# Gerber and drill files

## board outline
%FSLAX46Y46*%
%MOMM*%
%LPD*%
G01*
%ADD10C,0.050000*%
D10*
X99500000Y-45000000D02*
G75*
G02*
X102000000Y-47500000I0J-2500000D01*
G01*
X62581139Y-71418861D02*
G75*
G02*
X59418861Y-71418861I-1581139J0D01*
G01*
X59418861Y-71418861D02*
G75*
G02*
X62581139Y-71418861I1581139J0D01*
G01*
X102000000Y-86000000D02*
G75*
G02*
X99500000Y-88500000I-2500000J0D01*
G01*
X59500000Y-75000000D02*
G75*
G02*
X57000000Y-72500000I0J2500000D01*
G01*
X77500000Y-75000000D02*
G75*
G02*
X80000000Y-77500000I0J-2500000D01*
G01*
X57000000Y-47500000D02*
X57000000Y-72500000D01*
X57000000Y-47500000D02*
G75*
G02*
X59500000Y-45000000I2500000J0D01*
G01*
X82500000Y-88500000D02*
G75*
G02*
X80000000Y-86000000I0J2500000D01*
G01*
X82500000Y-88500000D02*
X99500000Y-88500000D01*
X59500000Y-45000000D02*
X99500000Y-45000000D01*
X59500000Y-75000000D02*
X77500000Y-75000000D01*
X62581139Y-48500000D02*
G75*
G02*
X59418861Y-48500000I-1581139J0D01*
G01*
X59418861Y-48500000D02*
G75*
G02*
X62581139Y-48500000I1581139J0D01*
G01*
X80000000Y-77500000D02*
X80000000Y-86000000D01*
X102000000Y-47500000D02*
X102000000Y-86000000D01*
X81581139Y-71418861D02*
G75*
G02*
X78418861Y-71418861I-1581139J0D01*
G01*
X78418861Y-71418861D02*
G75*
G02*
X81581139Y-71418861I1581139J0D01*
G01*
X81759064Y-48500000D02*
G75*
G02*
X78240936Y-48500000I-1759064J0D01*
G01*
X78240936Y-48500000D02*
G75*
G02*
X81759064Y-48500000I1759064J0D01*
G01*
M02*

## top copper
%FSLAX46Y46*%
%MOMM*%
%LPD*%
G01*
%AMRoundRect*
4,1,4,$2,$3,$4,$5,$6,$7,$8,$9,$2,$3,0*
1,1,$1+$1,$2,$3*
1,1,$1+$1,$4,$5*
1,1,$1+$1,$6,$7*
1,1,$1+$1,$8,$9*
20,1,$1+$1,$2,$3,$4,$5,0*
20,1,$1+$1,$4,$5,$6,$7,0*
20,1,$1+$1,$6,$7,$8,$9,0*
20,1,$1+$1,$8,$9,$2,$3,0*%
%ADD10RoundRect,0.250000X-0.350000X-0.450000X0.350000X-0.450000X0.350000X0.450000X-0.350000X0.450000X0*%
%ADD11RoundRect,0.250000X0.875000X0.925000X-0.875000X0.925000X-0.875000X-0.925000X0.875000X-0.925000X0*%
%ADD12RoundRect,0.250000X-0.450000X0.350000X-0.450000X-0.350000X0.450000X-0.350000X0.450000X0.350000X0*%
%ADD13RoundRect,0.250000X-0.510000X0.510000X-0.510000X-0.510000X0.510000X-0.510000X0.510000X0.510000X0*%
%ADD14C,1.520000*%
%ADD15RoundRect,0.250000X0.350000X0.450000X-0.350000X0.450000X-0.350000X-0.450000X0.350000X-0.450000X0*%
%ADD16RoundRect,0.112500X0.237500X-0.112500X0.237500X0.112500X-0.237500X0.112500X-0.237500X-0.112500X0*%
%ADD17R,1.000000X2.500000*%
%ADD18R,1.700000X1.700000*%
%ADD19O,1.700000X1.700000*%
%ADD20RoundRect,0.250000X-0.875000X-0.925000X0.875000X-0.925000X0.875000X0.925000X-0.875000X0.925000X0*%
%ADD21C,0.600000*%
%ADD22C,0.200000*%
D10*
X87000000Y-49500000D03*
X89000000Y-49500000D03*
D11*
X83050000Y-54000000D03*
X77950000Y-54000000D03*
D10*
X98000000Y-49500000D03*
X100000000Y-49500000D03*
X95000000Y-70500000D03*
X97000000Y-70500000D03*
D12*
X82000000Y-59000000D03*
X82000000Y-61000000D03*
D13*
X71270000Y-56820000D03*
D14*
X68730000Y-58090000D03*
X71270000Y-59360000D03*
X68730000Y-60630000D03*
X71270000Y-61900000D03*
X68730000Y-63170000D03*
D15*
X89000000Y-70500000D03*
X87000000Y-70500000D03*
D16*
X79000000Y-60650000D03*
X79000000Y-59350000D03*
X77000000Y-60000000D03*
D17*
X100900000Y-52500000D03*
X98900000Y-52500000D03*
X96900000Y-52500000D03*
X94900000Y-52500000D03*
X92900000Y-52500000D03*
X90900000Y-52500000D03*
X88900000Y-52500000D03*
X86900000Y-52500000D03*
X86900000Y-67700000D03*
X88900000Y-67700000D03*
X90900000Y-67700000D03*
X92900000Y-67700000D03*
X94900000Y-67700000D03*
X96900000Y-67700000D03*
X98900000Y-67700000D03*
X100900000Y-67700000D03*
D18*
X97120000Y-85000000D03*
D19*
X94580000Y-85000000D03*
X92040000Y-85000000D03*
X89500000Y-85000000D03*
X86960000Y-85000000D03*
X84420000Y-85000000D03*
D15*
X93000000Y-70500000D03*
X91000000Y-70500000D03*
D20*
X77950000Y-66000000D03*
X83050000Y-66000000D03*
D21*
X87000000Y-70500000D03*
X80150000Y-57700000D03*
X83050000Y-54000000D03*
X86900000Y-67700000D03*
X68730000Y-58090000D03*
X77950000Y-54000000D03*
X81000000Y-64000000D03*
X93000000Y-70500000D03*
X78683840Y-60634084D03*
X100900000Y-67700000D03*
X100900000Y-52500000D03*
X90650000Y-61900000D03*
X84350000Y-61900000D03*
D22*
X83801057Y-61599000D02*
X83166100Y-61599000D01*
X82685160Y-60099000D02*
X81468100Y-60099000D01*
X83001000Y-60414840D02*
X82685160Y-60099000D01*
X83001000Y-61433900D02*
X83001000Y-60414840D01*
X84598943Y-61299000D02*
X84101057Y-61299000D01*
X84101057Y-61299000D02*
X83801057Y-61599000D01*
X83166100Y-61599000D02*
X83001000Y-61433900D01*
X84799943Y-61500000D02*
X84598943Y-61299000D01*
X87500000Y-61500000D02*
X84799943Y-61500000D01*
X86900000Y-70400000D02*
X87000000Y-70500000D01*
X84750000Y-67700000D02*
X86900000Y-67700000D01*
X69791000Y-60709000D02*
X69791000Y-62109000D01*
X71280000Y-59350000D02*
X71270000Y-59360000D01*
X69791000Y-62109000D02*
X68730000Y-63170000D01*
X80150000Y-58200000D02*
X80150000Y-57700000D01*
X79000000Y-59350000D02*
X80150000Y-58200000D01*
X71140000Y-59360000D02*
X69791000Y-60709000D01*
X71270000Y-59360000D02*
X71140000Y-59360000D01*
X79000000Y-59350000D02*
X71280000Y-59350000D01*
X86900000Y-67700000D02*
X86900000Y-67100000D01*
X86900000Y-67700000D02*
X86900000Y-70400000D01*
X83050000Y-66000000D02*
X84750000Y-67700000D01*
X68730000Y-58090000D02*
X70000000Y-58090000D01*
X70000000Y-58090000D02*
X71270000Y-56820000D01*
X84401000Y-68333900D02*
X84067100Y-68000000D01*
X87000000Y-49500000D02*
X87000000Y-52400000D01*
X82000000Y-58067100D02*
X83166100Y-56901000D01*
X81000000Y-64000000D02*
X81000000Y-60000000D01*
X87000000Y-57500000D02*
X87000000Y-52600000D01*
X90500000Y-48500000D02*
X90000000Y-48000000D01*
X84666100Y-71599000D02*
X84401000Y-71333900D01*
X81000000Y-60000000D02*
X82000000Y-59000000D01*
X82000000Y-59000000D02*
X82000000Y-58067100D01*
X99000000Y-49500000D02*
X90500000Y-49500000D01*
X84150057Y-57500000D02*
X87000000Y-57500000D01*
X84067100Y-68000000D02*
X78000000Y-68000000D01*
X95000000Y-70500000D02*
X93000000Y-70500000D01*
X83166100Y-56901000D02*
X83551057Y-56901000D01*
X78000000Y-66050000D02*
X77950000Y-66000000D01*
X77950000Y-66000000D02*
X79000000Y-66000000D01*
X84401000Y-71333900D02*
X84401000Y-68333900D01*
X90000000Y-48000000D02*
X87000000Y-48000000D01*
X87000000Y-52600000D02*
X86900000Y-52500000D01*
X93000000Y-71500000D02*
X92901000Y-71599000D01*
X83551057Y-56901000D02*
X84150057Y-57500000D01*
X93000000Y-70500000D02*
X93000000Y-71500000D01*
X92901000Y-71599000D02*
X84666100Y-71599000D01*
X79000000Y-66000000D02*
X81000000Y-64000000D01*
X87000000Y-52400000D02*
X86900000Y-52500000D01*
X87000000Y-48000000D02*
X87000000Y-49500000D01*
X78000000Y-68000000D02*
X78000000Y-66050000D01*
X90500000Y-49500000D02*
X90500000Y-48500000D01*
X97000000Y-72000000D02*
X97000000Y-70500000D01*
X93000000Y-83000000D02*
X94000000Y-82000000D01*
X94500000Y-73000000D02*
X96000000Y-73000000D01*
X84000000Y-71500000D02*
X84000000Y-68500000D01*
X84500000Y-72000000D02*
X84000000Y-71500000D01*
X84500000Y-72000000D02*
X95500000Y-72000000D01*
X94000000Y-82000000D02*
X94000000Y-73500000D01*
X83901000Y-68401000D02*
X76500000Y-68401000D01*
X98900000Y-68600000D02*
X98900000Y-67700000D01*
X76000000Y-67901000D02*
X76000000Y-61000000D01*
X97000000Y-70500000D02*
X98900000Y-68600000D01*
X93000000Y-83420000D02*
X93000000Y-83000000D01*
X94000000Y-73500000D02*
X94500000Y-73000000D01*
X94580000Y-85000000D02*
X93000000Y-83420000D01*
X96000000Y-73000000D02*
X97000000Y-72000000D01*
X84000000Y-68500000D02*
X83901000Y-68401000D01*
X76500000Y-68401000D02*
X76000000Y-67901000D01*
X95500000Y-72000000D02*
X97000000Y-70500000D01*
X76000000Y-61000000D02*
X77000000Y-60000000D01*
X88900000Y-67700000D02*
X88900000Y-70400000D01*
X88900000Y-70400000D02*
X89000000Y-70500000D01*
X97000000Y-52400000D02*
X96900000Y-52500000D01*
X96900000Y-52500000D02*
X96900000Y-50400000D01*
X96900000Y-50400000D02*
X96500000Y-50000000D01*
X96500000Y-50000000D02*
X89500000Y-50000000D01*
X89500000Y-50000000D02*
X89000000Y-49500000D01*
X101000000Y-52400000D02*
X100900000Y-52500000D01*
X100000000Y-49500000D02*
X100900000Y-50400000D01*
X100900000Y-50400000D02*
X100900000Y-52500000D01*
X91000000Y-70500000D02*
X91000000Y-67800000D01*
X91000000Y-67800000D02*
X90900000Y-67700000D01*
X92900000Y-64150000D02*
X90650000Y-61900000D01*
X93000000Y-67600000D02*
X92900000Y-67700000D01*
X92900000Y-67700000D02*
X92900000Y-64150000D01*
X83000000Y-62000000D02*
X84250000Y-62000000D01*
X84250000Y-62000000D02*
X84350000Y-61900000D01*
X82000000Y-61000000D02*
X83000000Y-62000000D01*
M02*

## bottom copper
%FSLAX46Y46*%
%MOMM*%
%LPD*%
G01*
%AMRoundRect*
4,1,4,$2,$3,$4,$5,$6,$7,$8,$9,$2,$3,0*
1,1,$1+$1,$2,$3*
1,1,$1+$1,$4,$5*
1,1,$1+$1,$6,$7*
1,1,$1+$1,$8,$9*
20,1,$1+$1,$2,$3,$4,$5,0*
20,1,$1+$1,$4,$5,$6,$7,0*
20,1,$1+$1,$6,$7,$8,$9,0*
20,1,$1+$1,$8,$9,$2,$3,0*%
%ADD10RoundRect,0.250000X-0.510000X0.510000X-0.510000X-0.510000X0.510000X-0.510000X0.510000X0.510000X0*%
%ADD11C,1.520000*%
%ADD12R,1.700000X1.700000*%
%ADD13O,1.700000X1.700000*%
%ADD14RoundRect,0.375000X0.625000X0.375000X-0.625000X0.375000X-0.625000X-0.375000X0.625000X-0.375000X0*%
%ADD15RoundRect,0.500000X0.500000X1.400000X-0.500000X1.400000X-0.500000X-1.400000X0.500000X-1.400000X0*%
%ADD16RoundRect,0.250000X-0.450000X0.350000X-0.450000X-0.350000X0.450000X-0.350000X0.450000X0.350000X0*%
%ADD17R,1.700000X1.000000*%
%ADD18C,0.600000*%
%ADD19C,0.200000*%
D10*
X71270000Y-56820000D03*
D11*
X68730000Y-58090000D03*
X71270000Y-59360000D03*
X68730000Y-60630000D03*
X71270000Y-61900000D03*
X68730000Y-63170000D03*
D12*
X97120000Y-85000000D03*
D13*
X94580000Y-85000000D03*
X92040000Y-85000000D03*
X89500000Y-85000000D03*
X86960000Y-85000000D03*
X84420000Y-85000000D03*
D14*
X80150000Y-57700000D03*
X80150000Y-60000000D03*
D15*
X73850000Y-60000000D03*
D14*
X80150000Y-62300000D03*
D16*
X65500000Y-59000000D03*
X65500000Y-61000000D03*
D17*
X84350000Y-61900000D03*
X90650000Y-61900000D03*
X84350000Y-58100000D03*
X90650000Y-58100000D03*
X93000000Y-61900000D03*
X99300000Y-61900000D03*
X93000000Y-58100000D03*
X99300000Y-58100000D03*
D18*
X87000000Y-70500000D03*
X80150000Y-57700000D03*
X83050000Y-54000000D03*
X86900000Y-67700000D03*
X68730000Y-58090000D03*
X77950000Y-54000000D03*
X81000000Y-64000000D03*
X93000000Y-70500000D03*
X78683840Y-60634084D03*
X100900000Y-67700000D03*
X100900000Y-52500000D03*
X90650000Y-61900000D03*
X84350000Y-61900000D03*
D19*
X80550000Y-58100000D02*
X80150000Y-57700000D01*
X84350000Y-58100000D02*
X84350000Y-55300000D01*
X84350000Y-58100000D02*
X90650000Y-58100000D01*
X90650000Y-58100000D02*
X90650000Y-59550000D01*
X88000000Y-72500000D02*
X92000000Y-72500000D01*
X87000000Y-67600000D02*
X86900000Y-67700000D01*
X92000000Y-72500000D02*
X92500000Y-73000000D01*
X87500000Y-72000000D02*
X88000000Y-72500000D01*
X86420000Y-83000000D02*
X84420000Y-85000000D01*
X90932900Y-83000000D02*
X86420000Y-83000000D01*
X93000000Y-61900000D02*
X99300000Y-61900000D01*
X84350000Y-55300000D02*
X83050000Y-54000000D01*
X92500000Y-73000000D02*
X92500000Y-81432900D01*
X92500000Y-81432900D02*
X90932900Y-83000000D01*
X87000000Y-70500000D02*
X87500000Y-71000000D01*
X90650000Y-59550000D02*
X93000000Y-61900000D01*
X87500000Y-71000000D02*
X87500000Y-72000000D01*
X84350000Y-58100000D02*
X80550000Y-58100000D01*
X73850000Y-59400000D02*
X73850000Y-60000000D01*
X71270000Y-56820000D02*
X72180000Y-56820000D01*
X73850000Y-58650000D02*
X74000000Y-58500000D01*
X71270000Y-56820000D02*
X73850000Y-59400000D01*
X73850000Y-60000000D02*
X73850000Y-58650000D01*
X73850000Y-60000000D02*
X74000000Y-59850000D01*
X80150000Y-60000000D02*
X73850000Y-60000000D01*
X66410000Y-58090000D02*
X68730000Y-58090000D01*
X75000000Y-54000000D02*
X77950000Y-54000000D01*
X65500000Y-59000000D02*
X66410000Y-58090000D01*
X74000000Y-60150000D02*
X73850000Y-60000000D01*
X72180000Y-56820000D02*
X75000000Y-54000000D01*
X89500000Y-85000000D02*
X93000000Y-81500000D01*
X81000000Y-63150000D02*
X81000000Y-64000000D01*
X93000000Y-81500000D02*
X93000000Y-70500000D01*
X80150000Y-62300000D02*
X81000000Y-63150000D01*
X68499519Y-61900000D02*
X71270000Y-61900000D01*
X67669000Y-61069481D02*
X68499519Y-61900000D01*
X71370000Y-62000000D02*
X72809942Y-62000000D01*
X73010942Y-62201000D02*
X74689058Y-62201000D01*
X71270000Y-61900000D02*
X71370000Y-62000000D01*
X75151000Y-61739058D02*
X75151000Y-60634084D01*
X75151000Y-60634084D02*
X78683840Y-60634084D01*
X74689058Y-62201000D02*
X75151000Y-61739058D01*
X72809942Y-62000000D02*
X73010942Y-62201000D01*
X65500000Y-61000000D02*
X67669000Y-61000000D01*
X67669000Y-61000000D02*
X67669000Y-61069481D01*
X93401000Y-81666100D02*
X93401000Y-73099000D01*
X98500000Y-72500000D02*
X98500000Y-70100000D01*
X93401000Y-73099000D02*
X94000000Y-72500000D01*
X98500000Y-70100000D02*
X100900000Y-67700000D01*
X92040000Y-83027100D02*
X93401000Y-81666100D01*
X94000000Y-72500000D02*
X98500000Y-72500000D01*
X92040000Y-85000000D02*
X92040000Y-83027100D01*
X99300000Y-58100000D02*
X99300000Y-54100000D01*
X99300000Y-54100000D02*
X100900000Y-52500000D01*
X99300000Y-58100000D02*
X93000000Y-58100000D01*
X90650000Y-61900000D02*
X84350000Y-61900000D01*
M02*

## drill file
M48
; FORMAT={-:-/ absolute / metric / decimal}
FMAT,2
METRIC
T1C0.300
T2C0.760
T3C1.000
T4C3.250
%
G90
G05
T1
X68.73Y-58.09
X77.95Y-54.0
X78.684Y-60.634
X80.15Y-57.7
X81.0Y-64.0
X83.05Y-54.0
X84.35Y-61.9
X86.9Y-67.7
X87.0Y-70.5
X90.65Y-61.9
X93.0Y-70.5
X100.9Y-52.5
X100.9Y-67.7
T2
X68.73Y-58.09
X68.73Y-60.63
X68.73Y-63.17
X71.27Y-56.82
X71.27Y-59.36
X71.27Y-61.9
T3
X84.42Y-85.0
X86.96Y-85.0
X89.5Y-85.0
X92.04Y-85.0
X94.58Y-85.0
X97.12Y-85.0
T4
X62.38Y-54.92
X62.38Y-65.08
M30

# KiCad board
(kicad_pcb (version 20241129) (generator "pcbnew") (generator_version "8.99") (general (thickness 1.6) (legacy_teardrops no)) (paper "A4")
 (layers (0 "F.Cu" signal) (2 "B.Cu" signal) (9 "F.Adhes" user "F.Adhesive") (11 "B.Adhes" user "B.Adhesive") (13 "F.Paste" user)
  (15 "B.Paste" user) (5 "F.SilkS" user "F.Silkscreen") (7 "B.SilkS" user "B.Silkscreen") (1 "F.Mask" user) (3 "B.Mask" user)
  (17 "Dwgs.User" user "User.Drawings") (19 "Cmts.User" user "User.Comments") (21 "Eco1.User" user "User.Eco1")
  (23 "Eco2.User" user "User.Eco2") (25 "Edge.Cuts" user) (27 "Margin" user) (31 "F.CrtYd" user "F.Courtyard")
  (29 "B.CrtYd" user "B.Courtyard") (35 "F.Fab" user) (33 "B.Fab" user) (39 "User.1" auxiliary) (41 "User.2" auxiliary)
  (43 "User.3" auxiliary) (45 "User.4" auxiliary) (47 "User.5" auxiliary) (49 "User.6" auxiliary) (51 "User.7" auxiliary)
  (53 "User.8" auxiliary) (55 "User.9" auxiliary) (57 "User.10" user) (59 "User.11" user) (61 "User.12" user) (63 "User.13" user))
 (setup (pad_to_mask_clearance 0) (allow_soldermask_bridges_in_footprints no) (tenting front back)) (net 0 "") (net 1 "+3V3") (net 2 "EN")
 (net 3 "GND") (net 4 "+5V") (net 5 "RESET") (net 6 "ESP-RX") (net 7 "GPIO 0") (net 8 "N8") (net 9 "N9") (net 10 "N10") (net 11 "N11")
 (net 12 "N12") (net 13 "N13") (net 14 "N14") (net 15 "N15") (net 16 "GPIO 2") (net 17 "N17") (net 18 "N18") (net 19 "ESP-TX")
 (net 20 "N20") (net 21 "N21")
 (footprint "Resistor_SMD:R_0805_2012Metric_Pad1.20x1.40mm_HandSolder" (layer "F.Cu") (at 88 49.5)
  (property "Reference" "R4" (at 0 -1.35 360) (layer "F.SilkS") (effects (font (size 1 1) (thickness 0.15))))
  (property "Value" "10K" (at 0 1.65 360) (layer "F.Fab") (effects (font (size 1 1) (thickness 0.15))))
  (pad "1" smd roundrect (at -1 0) (size 1.2 1.4) (layers "F.Cu" "F.Mask" "F.Paste") (roundrect_rratio 0.208333) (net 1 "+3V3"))
  (pad "2" smd roundrect (at 1 0) (size 1.2 1.4) (layers "F.Cu" "F.Mask" "F.Paste") (roundrect_rratio 0.208333) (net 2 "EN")))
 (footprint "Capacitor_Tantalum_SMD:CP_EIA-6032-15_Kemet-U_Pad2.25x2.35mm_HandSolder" (layer "F.Cu") (at 80.5 54 180)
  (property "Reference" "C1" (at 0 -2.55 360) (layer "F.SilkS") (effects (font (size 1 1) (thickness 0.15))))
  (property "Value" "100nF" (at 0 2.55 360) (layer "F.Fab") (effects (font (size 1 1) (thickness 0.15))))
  (pad "1" smd roundrect (at -2.55 0 180) (size 2.25 2.35) (layers "F.Cu" "F.Mask" "F.Paste") (roundrect_rratio 0.111111) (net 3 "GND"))
  (pad "2" smd roundrect (at 2.55 0 180) (size 2.25 2.35) (layers "F.Cu" "F.Mask" "F.Paste") (roundrect_rratio 0.111111) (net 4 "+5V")))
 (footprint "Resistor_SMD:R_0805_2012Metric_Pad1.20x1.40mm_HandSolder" (layer "F.Cu") (at 99 49.5)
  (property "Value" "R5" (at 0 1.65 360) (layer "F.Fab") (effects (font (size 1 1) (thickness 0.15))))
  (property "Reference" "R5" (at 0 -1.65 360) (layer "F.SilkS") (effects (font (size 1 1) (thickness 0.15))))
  (pad "1" smd roundrect (at -1 0) (size 1.2 1.4) (layers "F.Cu" "F.Mask" "F.Paste") (roundrect_rratio 0.208333) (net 1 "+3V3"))
  (pad "2" smd roundrect (at 1 0) (size 1.2 1.4) (layers "F.Cu" "F.Mask" "F.Paste") (roundrect_rratio 0.208333) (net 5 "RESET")))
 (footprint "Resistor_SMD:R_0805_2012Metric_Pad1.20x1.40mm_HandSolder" (layer "F.Cu") (at 96 70.5)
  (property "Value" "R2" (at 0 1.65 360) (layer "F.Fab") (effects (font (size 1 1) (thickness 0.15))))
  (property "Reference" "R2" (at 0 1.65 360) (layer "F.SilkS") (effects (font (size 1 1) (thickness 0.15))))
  (pad "1" smd roundrect (at -1 0) (size 1.2 1.4) (layers "F.Cu" "F.Mask" "F.Paste") (roundrect_rratio 0.208333) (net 1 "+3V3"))
  (pad "2" smd roundrect (at 1 0) (size 1.2 1.4) (layers "F.Cu" "F.Mask" "F.Paste") (roundrect_rratio 0.208333) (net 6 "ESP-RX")))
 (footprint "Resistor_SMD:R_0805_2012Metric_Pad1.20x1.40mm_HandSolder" (layer "F.Cu") (at 82 60 -90)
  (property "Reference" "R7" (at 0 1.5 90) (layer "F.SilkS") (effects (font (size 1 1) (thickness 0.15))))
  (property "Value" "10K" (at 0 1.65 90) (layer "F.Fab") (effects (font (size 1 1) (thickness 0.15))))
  (pad "1" smd roundrect (at -1 0 270) (size 1.2 1.4) (layers "F.Cu" "F.Mask" "F.Paste") (roundrect_rratio 0.208333) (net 1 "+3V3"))
  (pad "2" smd roundrect (at 1 0 270) (size 1.2 1.4) (layers "F.Cu" "F.Mask" "F.Paste") (roundrect_rratio 0.208333) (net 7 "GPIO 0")))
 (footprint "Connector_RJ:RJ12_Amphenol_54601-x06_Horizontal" (layer "F.Cu") (at 71.27 56.82 -90)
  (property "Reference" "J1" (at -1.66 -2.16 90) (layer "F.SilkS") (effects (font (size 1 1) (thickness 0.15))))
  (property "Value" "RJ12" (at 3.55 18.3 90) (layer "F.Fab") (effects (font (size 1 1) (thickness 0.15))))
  (pad "" np_thru_hole circle (at -1.9 8.89 270) (size 3.25 3.25) (drill 3.25) (layers "*.Cu" "*.Mask"))
  (pad "" np_thru_hole circle (at 8.26 8.89 270) (size 3.25 3.25) (drill 3.25) (layers "*.Cu" "*.Mask"))
  (pad "1" thru_hole roundrect (at 0 0 270) (size 1.52 1.52) (drill 0.76) (layers "*.Cu" "*.Mask") (remove_unused_layers no)
   (roundrect_rratio 0.1644736842) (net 4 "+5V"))
  (pad "2" thru_hole circle (at 1.27 2.54 270) (size 1.52 1.52) (drill 0.76) (layers "*.Cu" "*.Mask") (remove_unused_layers no)
   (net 4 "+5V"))
  (pad "3" thru_hole circle (at 2.54 0 270) (size 1.52 1.52) (drill 0.76) (layers "*.Cu" "*.Mask") (remove_unused_layers no) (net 3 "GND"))
  (pad "4" thru_hole circle (at 3.81 2.54 270) (size 1.52 1.52) (drill 0.76) (layers "*.Cu" "*.Mask") (remove_unused_layers no) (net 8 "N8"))
  (pad "5" thru_hole circle (at 5.08 0 270) (size 1.52 1.52) (drill 0.76) (layers "*.Cu" "*.Mask") (remove_unused_layers no) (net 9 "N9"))
  (pad "6" thru_hole circle (at 6.35 2.54 270) (size 1.52 1.52) (drill 0.76) (layers "*.Cu" "*.Mask") (remove_unused_layers no)
   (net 3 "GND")))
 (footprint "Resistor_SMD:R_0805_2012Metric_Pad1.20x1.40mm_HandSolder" (layer "F.Cu") (at 88 70.5 180)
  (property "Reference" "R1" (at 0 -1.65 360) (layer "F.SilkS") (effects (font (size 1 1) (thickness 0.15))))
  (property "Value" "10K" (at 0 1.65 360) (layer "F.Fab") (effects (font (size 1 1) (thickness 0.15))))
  (pad "1" smd roundrect (at -1 0 180) (size 1.2 1.4) (layers "F.Cu" "F.Mask" "F.Paste") (roundrect_rratio 0.208333) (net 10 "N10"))
  (pad "2" smd roundrect (at 1 0 180) (size 1.2 1.4) (layers "F.Cu" "F.Mask" "F.Paste") (roundrect_rratio 0.208333) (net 3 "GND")))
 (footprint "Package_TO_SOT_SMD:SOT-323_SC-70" (layer "F.Cu") (at 78 60 180)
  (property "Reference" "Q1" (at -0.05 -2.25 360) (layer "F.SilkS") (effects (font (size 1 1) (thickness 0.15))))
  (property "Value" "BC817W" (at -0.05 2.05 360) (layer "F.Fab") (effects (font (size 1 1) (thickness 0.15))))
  (pad "1" smd roundrect (at -1 -0.65 90) (size 0.45 0.7) (layers "F.Cu" "F.Mask" "F.Paste") (roundrect_rratio 0.25) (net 9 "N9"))
  (pad "2" smd roundrect (at -1 0.65 90) (size 0.45 0.7) (layers "F.Cu" "F.Mask" "F.Paste") (roundrect_rratio 0.25) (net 3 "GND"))
  (pad "3" smd roundrect (at 1 0 90) (size 0.45 0.7) (layers "F.Cu" "F.Mask" "F.Paste") (roundrect_rratio 0.25) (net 6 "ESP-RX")))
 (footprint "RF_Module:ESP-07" (layer "F.Cu") (at 96 60.1 -90)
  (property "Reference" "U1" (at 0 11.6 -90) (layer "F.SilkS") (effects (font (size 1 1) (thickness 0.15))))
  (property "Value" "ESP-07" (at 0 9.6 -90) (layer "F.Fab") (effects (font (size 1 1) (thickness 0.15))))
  (pad "1" smd rect (at -7.6 -4.9 270) (size 2.5 1) (layers "F.Cu" "F.Mask" "F.Paste") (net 5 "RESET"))
  (pad "2" smd rect (at -7.6 -2.9 270) (size 2.5 1) (layers "F.Cu" "F.Mask" "F.Paste") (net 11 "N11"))
  (pad "3" smd rect (at -7.6 -0.9 270) (size 2.5 1) (layers "F.Cu" "F.Mask" "F.Paste") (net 2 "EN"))
  (pad "4" smd rect (at -7.6 1.1 270) (size 2.5 1) (layers "F.Cu" "F.Mask" "F.Paste") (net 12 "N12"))
  (pad "5" smd rect (at -7.6 3.1 270) (size 2.5 1) (layers "F.Cu" "F.Mask" "F.Paste") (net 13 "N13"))
  (pad "6" smd rect (at -7.6 5.1 270) (size 2.5 1) (layers "F.Cu" "F.Mask" "F.Paste") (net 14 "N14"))
  (pad "7" smd rect (at -7.6 7.1 270) (size 2.5 1) (layers "F.Cu" "F.Mask" "F.Paste") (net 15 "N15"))
  (pad "8" smd rect (at -7.6 9.1 270) (size 2.5 1) (layers "F.Cu" "F.Mask" "F.Paste") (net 1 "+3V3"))
  (pad "9" smd rect (at 7.6 9.1 270) (size 2.5 1) (layers "F.Cu" "F.Mask" "F.Paste") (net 3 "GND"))
  (pad "10" smd rect (at 7.6 7.1 270) (size 2.5 1) (layers "F.Cu" "F.Mask" "F.Paste") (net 10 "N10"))
  (pad "11" smd rect (at 7.6 5.1 270) (size 2.5 1) (layers "F.Cu" "F.Mask" "F.Paste") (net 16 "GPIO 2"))
  (pad "12" smd rect (at 7.6 3.1 270) (size 2.5 1) (layers "F.Cu" "F.Mask" "F.Paste") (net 7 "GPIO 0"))
  (pad "13" smd rect (at 7.6 1.1 270) (size 2.5 1) (layers "F.Cu" "F.Mask" "F.Paste") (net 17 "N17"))
  (pad "14" smd rect (at 7.6 -0.9 270) (size 2.5 1) (layers "F.Cu" "F.Mask" "F.Paste") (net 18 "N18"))
  (pad "15" smd rect (at 7.6 -2.9 270) (size 2.5 1) (layers "F.Cu" "F.Mask" "F.Paste") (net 6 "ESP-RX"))
  (pad "16" smd rect (at 7.6 -4.9 270) (size 2.5 1) (layers "F.Cu" "F.Mask" "F.Paste") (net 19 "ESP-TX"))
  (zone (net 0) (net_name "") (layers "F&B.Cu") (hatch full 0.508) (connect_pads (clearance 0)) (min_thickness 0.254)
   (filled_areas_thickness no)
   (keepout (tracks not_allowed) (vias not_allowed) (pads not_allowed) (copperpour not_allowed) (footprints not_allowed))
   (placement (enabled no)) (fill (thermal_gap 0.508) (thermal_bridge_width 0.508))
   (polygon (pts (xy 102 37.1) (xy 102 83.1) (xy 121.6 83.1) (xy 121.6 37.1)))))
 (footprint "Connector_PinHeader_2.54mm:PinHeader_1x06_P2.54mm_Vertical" (layer "F.Cu") (at 97.12 85 -90)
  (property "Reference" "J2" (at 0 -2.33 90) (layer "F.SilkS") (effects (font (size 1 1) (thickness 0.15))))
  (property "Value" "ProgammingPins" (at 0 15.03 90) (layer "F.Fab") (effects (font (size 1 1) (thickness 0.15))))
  (pad "1" thru_hole rect (at 0 0 270) (size 1.7 1.7) (drill 1) (layers "*.Cu" "*.Mask") (remove_unused_layers no) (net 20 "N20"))
  (pad "2" thru_hole oval (at 0 2.54 270) (size 1.7 1.7) (drill 1) (layers "*.Cu" "*.Mask") (remove_unused_layers no) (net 6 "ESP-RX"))
  (pad "3" thru_hole oval (at 0 5.08 270) (size 1.7 1.7) (drill 1) (layers "*.Cu" "*.Mask") (remove_unused_layers no) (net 19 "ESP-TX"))
  (pad "4" thru_hole oval (at 0 7.62 270) (size 1.7 1.7) (drill 1) (layers "*.Cu" "*.Mask") (remove_unused_layers no) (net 1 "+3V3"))
  (pad "5" thru_hole oval (at 0 10.16 270) (size 1.7 1.7) (drill 1) (layers "*.Cu" "*.Mask") (remove_unused_layers no) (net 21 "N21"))
  (pad "6" thru_hole oval (at 0 12.7 270) (size 1.7 1.7) (drill 1) (layers "*.Cu" "*.Mask") (remove_unused_layers no) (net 3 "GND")))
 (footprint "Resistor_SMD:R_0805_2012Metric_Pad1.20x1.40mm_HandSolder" (layer "F.Cu") (at 92 70.5 180)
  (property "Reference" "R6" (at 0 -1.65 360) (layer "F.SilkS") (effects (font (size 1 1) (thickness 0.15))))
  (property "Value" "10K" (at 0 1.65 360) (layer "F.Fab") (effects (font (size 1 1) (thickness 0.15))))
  (pad "1" smd roundrect (at -1 0 180) (size 1.2 1.4) (layers "F.Cu" "F.Mask" "F.Paste") (roundrect_rratio 0.208333) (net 1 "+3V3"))
  (pad "2" smd roundrect (at 1 0 180) (size 1.2 1.4) (layers "F.Cu" "F.Mask" "F.Paste") (roundrect_rratio 0.208333) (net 16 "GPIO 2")))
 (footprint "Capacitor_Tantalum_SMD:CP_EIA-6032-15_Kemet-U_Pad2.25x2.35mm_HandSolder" (layer "F.Cu") (at 80.5 66)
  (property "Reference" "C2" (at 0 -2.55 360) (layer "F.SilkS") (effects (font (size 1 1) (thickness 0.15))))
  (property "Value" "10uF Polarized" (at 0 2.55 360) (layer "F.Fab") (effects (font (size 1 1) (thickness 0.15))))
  (pad "1" smd roundrect (at -2.55 0) (size 2.25 2.35) (layers "F.Cu" "F.Mask" "F.Paste") (roundrect_rratio 0.111111) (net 1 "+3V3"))
  (pad "2" smd roundrect (at 2.55 0) (size 2.25 2.35) (layers "F.Cu" "F.Mask" "F.Paste") (roundrect_rratio 0.111111) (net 3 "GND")))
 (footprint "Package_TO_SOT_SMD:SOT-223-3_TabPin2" (layer "B.Cu") (at 77 60 180)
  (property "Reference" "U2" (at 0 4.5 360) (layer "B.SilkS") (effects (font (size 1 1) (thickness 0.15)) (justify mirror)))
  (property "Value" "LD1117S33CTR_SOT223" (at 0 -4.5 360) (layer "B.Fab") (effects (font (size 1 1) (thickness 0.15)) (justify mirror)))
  (pad "1" smd roundrect (at -3.15 2.3 180) (size 2 1.5) (layers "B.Cu" "B.Mask" "B.Paste") (roundrect_rratio 0.25) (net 3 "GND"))
  (pad "2" smd roundrect (at -3.15 0 180) (size 2 1.5) (layers "B.Cu" "B.Mask" "B.Paste") (roundrect_rratio 0.25) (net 4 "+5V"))
  (pad "2" smd roundrect (at 3.15 0 180) (size 2 3.8) (layers "B.Cu" "B.Mask" "B.Paste") (roundrect_rratio 0.25) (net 4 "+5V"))
  (pad "3" smd roundrect (at -3.15 -2.3 180) (size 2 1.5) (layers "B.Cu" "B.Mask" "B.Paste") (roundrect_rratio 0.25) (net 1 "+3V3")))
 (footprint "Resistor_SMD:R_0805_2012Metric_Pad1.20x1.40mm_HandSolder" (layer "B.Cu") (at 65.5 60 -90)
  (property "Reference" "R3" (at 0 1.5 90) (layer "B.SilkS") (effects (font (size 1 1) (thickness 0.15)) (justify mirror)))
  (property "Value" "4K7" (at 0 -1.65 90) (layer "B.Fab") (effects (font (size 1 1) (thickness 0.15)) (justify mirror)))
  (pad "1" smd roundrect (at -1 0 270) (size 1.2 1.4) (layers "B.Cu" "B.Mask" "B.Paste") (roundrect_rratio 0.208333) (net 4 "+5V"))
  (pad "2" smd roundrect (at 1 0 270) (size 1.2 1.4) (layers "B.Cu" "B.Mask" "B.Paste") (roundrect_rratio 0.208333) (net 9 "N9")))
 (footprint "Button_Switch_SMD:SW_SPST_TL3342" (layer "B.Cu") (at 87.5 60)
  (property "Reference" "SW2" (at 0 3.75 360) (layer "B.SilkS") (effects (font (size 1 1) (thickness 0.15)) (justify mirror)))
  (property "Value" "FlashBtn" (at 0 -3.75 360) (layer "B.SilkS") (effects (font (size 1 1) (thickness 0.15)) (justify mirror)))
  (pad "1" smd rect (at -3.15 1.9) (size 1.7 1) (layers "B.Cu" "B.Mask" "B.Paste") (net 7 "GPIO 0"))
  (pad "1" smd rect (at 3.15 1.9) (size 1.7 1) (layers "B.Cu" "B.Mask" "B.Paste") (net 7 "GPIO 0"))
  (pad "2" smd rect (at -3.15 -1.9) (size 1.7 1) (layers "B.Cu" "B.Mask" "B.Paste") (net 3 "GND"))
  (pad "2" smd rect (at 3.15 -1.9) (size 1.7 1) (layers "B.Cu" "B.Mask" "B.Paste") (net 3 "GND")))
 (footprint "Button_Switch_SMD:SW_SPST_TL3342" (layer "B.Cu") (at 96.15 60)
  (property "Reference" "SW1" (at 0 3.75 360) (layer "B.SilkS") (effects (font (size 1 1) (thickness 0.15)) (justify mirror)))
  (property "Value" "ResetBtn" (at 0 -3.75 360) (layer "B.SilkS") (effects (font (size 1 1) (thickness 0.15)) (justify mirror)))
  (pad "1" smd rect (at -3.15 1.9) (size 1.7 1) (layers "B.Cu" "B.Mask" "B.Paste") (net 3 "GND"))
  (pad "1" smd rect (at 3.15 1.9) (size 1.7 1) (layers "B.Cu" "B.Mask" "B.Paste") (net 3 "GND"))
  (pad "2" smd rect (at -3.15 -1.9) (size 1.7 1) (layers "B.Cu" "B.Mask" "B.Paste") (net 5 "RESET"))
  (pad "2" smd rect (at 3.15 -1.9) (size 1.7 1) (layers "B.Cu" "B.Mask" "B.Paste") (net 5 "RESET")))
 (gr_arc (start 99.5 45) (mid 101.267767 45.732233) (end 102 47.5) (stroke (width 0.05) (type default)) (layer "Edge.Cuts"))
 (gr_circle (center 61 71.418861) (end 61.5 72.918861) (stroke (width 0.05) (type default)) (fill no) (layer "Edge.Cuts"))
 (gr_arc (start 102 86) (mid 101.267767 87.767767) (end 99.5 88.5) (stroke (width 0.05) (type default)) (layer "Edge.Cuts"))
 (gr_arc (start 59.5 75) (mid 57.732233 74.267767) (end 57 72.5) (stroke (width 0.05) (type default)) (layer "Edge.Cuts"))
 (gr_arc (start 77.5 75) (mid 79.267767 75.732233) (end 80 77.5) (stroke (width 0.05) (type default)) (layer "Edge.Cuts"))
 (gr_line (start 57 47.5) (end 57 72.5) (stroke (width 0.05) (type default)) (layer "Edge.Cuts"))
 (gr_arc (start 57 47.5) (mid 57.732233 45.732233) (end 59.5 45) (stroke (width 0.05) (type default)) (layer "Edge.Cuts"))
 (gr_arc (start 82.5 88.5) (mid 80.732233 87.767767) (end 80 86) (stroke (width 0.05) (type default)) (layer "Edge.Cuts"))
 (gr_line (start 82.5 88.5) (end 99.5 88.5) (stroke (width 0.05) (type default)) (layer "Edge.Cuts"))
 (gr_line (start 59.5 45) (end 99.5 45) (stroke (width 0.05) (type default)) (layer "Edge.Cuts"))
 (gr_line (start 59.5 75) (end 77.5 75) (stroke (width 0.05) (type default)) (layer "Edge.Cuts"))
 (gr_circle (center 61 48.5) (end 61.5 50) (stroke (width 0.05) (type default)) (fill no) (layer "Edge.Cuts"))
 (gr_line (start 80 77.5) (end 80 86) (stroke (width 0.05) (type default)) (layer "Edge.Cuts"))
 (gr_line (start 102 47.5) (end 102 86) (stroke (width 0.05) (type default)) (layer "Edge.Cuts"))
 (gr_circle (center 80 71.418861) (end 80.5 72.918861) (stroke (width 0.05) (type default)) (fill no) (layer "Edge.Cuts"))
 (gr_circle (center 80 48.5) (end 80.918861 50) (stroke (width 0.05) (type default)) (fill no) (layer "Edge.Cuts"))
 (segment (start 83.801057 61.599) (end 83.1661 61.599) (width 0.2) (layer "F.Cu") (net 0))
 (segment (start 82.68516 60.099) (end 81.4681 60.099) (width 0.2) (layer "F.Cu") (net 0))
 (segment (start 83.001 60.41484) (end 82.68516 60.099) (width 0.2) (layer "F.Cu") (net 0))
 (segment (start 83.001 61.4339) (end 83.001 60.41484) (width 0.2) (layer "F.Cu") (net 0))
 (segment (start 84.598943 61.299) (end 84.101057 61.299) (width 0.2) (layer "F.Cu") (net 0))
 (segment (start 84.101057 61.299) (end 83.801057 61.599) (width 0.2) (layer "F.Cu") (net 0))
 (segment (start 83.1661 61.599) (end 83.001 61.4339) (width 0.2) (layer "F.Cu") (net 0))
 (segment (start 84.799943 61.5) (end 84.598943 61.299) (width 0.2) (layer "F.Cu") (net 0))
 (segment (start 87.5 61.5) (end 84.799943 61.5) (width 0.2) (layer "F.Cu") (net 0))
 (segment (start 86.9 70.4) (end 87 70.5) (width 0.2) (layer "F.Cu") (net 3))
 (segment (start 84.75 67.7) (end 86.9 67.7) (width 0.2) (layer "F.Cu") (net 3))
 (segment (start 69.791 60.709) (end 69.791 62.109) (width 0.2) (layer "F.Cu") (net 3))
 (segment (start 71.28 59.35) (end 71.27 59.36) (width 0.2) (layer "F.Cu") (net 3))
 (segment (start 69.791 62.109) (end 68.73 63.17) (width 0.2) (layer "F.Cu") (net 3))
 (segment (start 80.15 58.2) (end 80.15 57.7) (width 0.2) (layer "F.Cu") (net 3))
 (segment (start 79 59.35) (end 80.15 58.2) (width 0.2) (layer "F.Cu") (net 3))
 (segment (start 71.14 59.36) (end 69.791 60.709) (width 0.2) (layer "F.Cu") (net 3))
 (segment (start 71.27 59.36) (end 71.14 59.36) (width 0.2) (layer "F.Cu") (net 3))
 (segment (start 79 59.35) (end 71.28 59.35) (width 0.2) (layer "F.Cu") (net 3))
 (segment (start 86.9 67.7) (end 86.9 67.1) (width 0.2) (layer "F.Cu") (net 3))
 (segment (start 86.9 67.7) (end 86.9 70.4) (width 0.2) (layer "F.Cu") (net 3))
 (segment (start 83.05 66) (end 84.75 67.7) (width 0.2) (layer "F.Cu") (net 3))
 (via (at 87 70.5) (size 0.6) (drill 0.3) (layers "F.Cu" "B.Cu") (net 3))
 (via (at 80.15 57.7) (size 0.6) (drill 0.3) (layers "F.Cu" "B.Cu") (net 3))
 (via (at 83.05 54) (size 0.6) (drill 0.3) (layers "F.Cu" "B.Cu") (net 3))
 (via (at 86.9 67.7) (size 0.6) (drill 0.3) (layers "F.Cu" "B.Cu") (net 3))
 (segment (start 80.55 58.1) (end 80.15 57.7) (width 0.2) (layer "B.Cu") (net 3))
 (segment (start 84.35 58.1) (end 84.35 55.3) (width 0.2) (layer "B.Cu") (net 3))
 (segment (start 84.35 58.1) (end 90.65 58.1) (width 0.2) (layer "B.Cu") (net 3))
 (segment (start 90.65 58.1) (end 90.65 59.55) (width 0.2) (layer "B.Cu") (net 3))
 (segment (start 88 72.5) (end 92 72.5) (width 0.2) (layer "B.Cu") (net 3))
 (segment (start 87 67.6) (end 86.9 67.7) (width 0.2) (layer "B.Cu") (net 3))
 (segment (start 92 72.5) (end 92.5 73) (width 0.2) (layer "B.Cu") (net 3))
 (segment (start 87.5 72) (end 88 72.5) (width 0.2) (layer "B.Cu") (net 3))
 (segment (start 86.42 83) (end 84.42 85) (width 0.2) (layer "B.Cu") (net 3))
 (segment (start 90.9329 83) (end 86.42 83) (width 0.2) (layer "B.Cu") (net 3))
 (segment (start 93 61.9) (end 99.3 61.9) (width 0.2) (layer "B.Cu") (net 3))
 (segment (start 84.35 55.3) (end 83.05 54) (width 0.2) (layer "B.Cu") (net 3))
 (segment (start 92.5 73) (end 92.5 81.4329) (width 0.2) (layer "B.Cu") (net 3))
 (segment (start 92.5 81.4329) (end 90.9329 83) (width 0.2) (layer "B.Cu") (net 3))
 (segment (start 87 70.5) (end 87.5 71) (width 0.2) (layer "B.Cu") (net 3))
 (segment (start 90.65 59.55) (end 93 61.9) (width 0.2) (layer "B.Cu") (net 3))
 (segment (start 87.5 71) (end 87.5 72) (width 0.2) (layer "B.Cu") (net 3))
 (segment (start 84.35 58.1) (end 80.55 58.1) (width 0.2) (layer "B.Cu") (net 3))
 (segment (start 68.73 58.09) (end 70 58.09) (width 0.2) (layer "F.Cu") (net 4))
 (segment (start 70 58.09) (end 71.27 56.82) (width 0.2) (layer "F.Cu") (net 4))
 (via (at 68.73 58.09) (size 0.6) (drill 0.3) (layers "F.Cu" "B.Cu") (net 4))
 (via (at 77.95 54) (size 0.6) (drill 0.3) (layers "F.Cu" "B.Cu") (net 4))
 (segment (start 73.85 59.4) (end 73.85 60) (width 0.2) (layer "B.Cu") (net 4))
 (segment (start 71.27 56.82) (end 72.18 56.82) (width 0.2) (layer "B.Cu") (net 4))
 (segment (start 73.85 58.65) (end 74 58.5) (width 0.2) (layer "B.Cu") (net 4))
 (segment (start 71.27 56.82) (end 73.85 59.4) (width 0.2) (layer "B.Cu") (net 4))
 (segment (start 73.85 60) (end 73.85 58.65) (width 0.2) (layer "B.Cu") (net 4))
 (segment (start 73.85 60) (end 74 59.85) (width 0.2) (layer "B.Cu") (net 4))
 (segment (start 80.15 60) (end 73.85 60) (width 0.2) (layer "B.Cu") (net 4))
 (segment (start 66.41 58.09) (end 68.73 58.09) (width 0.2) (layer "B.Cu") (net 4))
 (segment (start 75 54) (end 77.95 54) (width 0.2) (layer "B.Cu") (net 4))
 (segment (start 65.5 59) (end 66.41 58.09) (width 0.2) (layer "B.Cu") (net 4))
 (segment (start 74 60.15) (end 73.85 60) (width 0.2) (layer "B.Cu") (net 4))
 (segment (start 72.18 56.82) (end 75 54) (width 0.2) (layer "B.Cu") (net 4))
 (segment (start 84.401 68.3339) (end 84.0671 68) (width 0.2) (layer "F.Cu") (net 1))
 (segment (start 87 49.5) (end 87 52.4) (width 0.2) (layer "F.Cu") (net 1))
 (segment (start 82 58.0671) (end 83.1661 56.901) (width 0.2) (layer "F.Cu") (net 1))
 (segment (start 81 64) (end 81 60) (width 0.2) (layer "F.Cu") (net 1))
 (segment (start 87 57.5) (end 87 52.6) (width 0.2) (layer "F.Cu") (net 1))
 (segment (start 90.5 48.5) (end 90 48) (width 0.2) (layer "F.Cu") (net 1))
 (segment (start 84.6661 71.599) (end 84.401 71.3339) (width 0.2) (layer "F.Cu") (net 1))
 (segment (start 81 60) (end 82 59) (width 0.2) (layer "F.Cu") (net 1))
 (segment (start 82 59) (end 82 58.0671) (width 0.2) (layer "F.Cu") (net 1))
 (segment (start 99 49.5) (end 90.5 49.5) (width 0.2) (layer "F.Cu") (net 1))
 (segment (start 84.150057 57.5) (end 87 57.5) (width 0.2) (layer "F.Cu") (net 1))
 (segment (start 84.0671 68) (end 78 68) (width 0.2) (layer "F.Cu") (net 1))
 (segment (start 95 70.5) (end 93 70.5) (width 0.2) (layer "F.Cu") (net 1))
 (segment (start 83.1661 56.901) (end 83.551057 56.901) (width 0.2) (layer "F.Cu") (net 1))
 (segment (start 78 66.05) (end 77.95 66) (width 0.2) (layer "F.Cu") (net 1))
 (segment (start 77.95 66) (end 79 66) (width 0.2) (layer "F.Cu") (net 1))
 (segment (start 84.401 71.3339) (end 84.401 68.3339) (width 0.2) (layer "F.Cu") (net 1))
 (segment (start 90 48) (end 87 48) (width 0.2) (layer "F.Cu") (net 1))
 (segment (start 87 52.6) (end 86.9 52.5) (width 0.2) (layer "F.Cu") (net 1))
 (segment (start 93 71.5) (end 92.901 71.599) (width 0.2) (layer "F.Cu") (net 1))
 (segment (start 83.551057 56.901) (end 84.150057 57.5) (width 0.2) (layer "F.Cu") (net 1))
 (segment (start 93 70.5) (end 93 71.5) (width 0.2) (layer "F.Cu") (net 1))
 (segment (start 92.901 71.599) (end 84.6661 71.599) (width 0.2) (layer "F.Cu") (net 1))
 (segment (start 79 66) (end 81 64) (width 0.2) (layer "F.Cu") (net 1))
 (segment (start 87 52.4) (end 86.9 52.5) (width 0.2) (layer "F.Cu") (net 1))
 (segment (start 87 48) (end 87 49.5) (width 0.2) (layer "F.Cu") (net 1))
 (segment (start 78 68) (end 78 66.05) (width 0.2) (layer "F.Cu") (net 1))
 (segment (start 90.5 49.5) (end 90.5 48.5) (width 0.2) (layer "F.Cu") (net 1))
 (via (at 81 64) (size 0.6) (drill 0.3) (layers "F.Cu" "B.Cu") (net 1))
 (via (at 93 70.5) (size 0.6) (drill 0.3) (layers "F.Cu" "B.Cu") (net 1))
 (segment (start 89.5 85) (end 93 81.5) (width 0.2) (layer "B.Cu") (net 1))
 (segment (start 81 63.15) (end 81 64) (width 0.2) (layer "B.Cu") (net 1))
 (segment (start 93 81.5) (end 93 70.5) (width 0.2) (layer "B.Cu") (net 1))
 (segment (start 80.15 62.3) (end 81 63.15) (width 0.2) (layer "B.Cu") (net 1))
 (via (at 78.68384 60.634084) (size 0.6) (drill 0.3) (layers "F.Cu" "B.Cu") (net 9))
 (segment (start 68.499519 61.9) (end 71.27 61.9) (width 0.2) (layer "B.Cu") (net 9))
 (segment (start 67.669 61.069481) (end 68.499519 61.9) (width 0.2) (layer "B.Cu") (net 9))
 (segment (start 71.37 62) (end 72.809942 62) (width 0.2) (layer "B.Cu") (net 9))
 (segment (start 73.010942 62.201) (end 74.689058 62.201) (width 0.2) (layer "B.Cu") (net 9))
 (segment (start 71.27 61.9) (end 71.37 62) (width 0.2) (layer "B.Cu") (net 9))
 (segment (start 75.151 61.739058) (end 75.151 60.634084) (width 0.2) (layer "B.Cu") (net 9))
 (segment (start 75.151 60.634084) (end 78.68384 60.634084) (width 0.2) (layer "B.Cu") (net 9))
 (segment (start 74.689058 62.201) (end 75.151 61.739058) (width 0.2) (layer "B.Cu") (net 9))
 (segment (start 72.809942 62) (end 73.010942 62.201) (width 0.2) (layer "B.Cu") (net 9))
 (segment (start 65.5 61) (end 67.669 61) (width 0.2) (layer "B.Cu") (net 9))
 (segment (start 67.669 61) (end 67.669 61.069481) (width 0.2) (layer "B.Cu") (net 9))
 (segment (start 97 72) (end 97 70.5) (width 0.2) (layer "F.Cu") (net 6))
 (segment (start 93 83) (end 94 82) (width 0.2) (layer "F.Cu") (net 6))
 (segment (start 94.5 73) (end 96 73) (width 0.2) (layer "F.Cu") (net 6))
 (segment (start 84 71.5) (end 84 68.5) (width 0.2) (layer "F.Cu") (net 6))
 (segment (start 84.5 72) (end 84 71.5) (width 0.2) (layer "F.Cu") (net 6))
 (segment (start 84.5 72) (end 95.5 72) (width 0.2) (layer "F.Cu") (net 6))
 (segment (start 94 82) (end 94 73.5) (width 0.2) (layer "F.Cu") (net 6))
 (segment (start 83.901 68.401) (end 76.5 68.401) (width 0.2) (layer "F.Cu") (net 6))
 (segment (start 98.9 68.6) (end 98.9 67.7) (width 0.2) (layer "F.Cu") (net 6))
 (segment (start 76 67.901) (end 76 61) (width 0.2) (layer "F.Cu") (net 6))
 (segment (start 97 70.5) (end 98.9 68.6) (width 0.2) (layer "F.Cu") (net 6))
 (segment (start 93 83.42) (end 93 83) (width 0.2) (layer "F.Cu") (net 6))
 (segment (start 94 73.5) (end 94.5 73) (width 0.2) (layer "F.Cu") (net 6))
 (segment (start 94.58 85) (end 93 83.42) (width 0.2) (layer "F.Cu") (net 6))
 (segment (start 96 73) (end 97 72) (width 0.2) (layer "F.Cu") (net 6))
 (segment (start 84 68.5) (end 83.901 68.401) (width 0.2) (layer "F.Cu") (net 6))
 (segment (start 76.5 68.401) (end 76 67.901) (width 0.2) (layer "F.Cu") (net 6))
 (segment (start 95.5 72) (end 97 70.5) (width 0.2) (layer "F.Cu") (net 6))
 (segment (start 76 61) (end 77 60) (width 0.2) (layer "F.Cu") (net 6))
 (via (at 100.9 67.7) (size 0.6) (drill 0.3) (layers "F.Cu" "B.Cu") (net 19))
 (segment (start 93.401 81.6661) (end 93.401 73.099) (width 0.2) (layer "B.Cu") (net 19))
 (segment (start 98.5 72.5) (end 98.5 70.1) (width 0.2) (layer "B.Cu") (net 19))
 (segment (start 93.401 73.099) (end 94 72.5) (width 0.2) (layer "B.Cu") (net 19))
 (segment (start 98.5 70.1) (end 100.9 67.7) (width 0.2) (layer "B.Cu") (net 19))
 (segment (start 92.04 83.0271) (end 93.401 81.6661) (width 0.2) (layer "B.Cu") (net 19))
 (segment (start 94 72.5) (end 98.5 72.5) (width 0.2) (layer "B.Cu") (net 19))
 (segment (start 92.04 85) (end 92.04 83.0271) (width 0.2) (layer "B.Cu") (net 19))
 (segment (start 88.9 67.7) (end 88.9 70.4) (width 0.2) (layer "F.Cu") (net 10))
 (segment (start 88.9 70.4) (end 89 70.5) (width 0.2) (layer "F.Cu") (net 10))
 (segment (start 97 52.4) (end 96.9 52.5) (width 0.2) (layer "F.Cu") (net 2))
 (segment (start 96.9 52.5) (end 96.9 50.4) (width 0.2) (layer "F.Cu") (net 2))
 (segment (start 96.9 50.4) (end 96.5 50) (width 0.2) (layer "F.Cu") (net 2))
 (segment (start 96.5 50) (end 89.5 50) (width 0.2) (layer "F.Cu") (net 2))
 (segment (start 89.5 50) (end 89 49.5) (width 0.2) (layer "F.Cu") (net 2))
 (segment (start 101 52.4) (end 100.9 52.5) (width 0.2) (layer "F.Cu") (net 5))
 (segment (start 100 49.5) (end 100.9 50.4) (width 0.2) (layer "F.Cu") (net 5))
 (segment (start 100.9 50.4) (end 100.9 52.5) (width 0.2) (layer "F.Cu") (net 5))
 (via (at 100.9 52.5) (size 0.6) (drill 0.3) (layers "F.Cu" "B.Cu") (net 5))
 (segment (start 99.3 58.1) (end 99.3 54.1) (width 0.2) (layer "B.Cu") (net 5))
 (segment (start 99.3 54.1) (end 100.9 52.5) (width 0.2) (layer "B.Cu") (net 5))
 (segment (start 99.3 58.1) (end 93 58.1) (width 0.2) (layer "B.Cu") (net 5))
 (segment (start 91 70.5) (end 91 67.8) (width 0.2) (layer "F.Cu") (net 16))
 (segment (start 91 67.8) (end 90.9 67.7) (width 0.2) (layer "F.Cu") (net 16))
 (segment (start 92.9 64.15) (end 90.65 61.9) (width 0.2) (layer "F.Cu") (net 7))
 (segment (start 93 67.6) (end 92.9 67.7) (width 0.2) (layer "F.Cu") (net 7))
 (segment (start 92.9 67.7) (end 92.9 64.15) (width 0.2) (layer "F.Cu") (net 7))
 (segment (start 83 62) (end 84.25 62) (width 0.2) (layer "F.Cu") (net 7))
 (segment (start 84.25 62) (end 84.35 61.9) (width 0.2) (layer "F.Cu") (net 7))
 (segment (start 82 61) (end 83 62) (width 0.2) (layer "F.Cu") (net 7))
 (via (at 90.65 61.9) (size 0.6) (drill 0.3) (layers "F.Cu" "B.Cu") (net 7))
 (via (at 84.35 61.9) (size 0.6) (drill 0.3) (layers "F.Cu" "B.Cu") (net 7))
 (segment (start 90.65 61.9) (end 84.35 61.9) (width 0.2) (layer "B.Cu") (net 7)))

